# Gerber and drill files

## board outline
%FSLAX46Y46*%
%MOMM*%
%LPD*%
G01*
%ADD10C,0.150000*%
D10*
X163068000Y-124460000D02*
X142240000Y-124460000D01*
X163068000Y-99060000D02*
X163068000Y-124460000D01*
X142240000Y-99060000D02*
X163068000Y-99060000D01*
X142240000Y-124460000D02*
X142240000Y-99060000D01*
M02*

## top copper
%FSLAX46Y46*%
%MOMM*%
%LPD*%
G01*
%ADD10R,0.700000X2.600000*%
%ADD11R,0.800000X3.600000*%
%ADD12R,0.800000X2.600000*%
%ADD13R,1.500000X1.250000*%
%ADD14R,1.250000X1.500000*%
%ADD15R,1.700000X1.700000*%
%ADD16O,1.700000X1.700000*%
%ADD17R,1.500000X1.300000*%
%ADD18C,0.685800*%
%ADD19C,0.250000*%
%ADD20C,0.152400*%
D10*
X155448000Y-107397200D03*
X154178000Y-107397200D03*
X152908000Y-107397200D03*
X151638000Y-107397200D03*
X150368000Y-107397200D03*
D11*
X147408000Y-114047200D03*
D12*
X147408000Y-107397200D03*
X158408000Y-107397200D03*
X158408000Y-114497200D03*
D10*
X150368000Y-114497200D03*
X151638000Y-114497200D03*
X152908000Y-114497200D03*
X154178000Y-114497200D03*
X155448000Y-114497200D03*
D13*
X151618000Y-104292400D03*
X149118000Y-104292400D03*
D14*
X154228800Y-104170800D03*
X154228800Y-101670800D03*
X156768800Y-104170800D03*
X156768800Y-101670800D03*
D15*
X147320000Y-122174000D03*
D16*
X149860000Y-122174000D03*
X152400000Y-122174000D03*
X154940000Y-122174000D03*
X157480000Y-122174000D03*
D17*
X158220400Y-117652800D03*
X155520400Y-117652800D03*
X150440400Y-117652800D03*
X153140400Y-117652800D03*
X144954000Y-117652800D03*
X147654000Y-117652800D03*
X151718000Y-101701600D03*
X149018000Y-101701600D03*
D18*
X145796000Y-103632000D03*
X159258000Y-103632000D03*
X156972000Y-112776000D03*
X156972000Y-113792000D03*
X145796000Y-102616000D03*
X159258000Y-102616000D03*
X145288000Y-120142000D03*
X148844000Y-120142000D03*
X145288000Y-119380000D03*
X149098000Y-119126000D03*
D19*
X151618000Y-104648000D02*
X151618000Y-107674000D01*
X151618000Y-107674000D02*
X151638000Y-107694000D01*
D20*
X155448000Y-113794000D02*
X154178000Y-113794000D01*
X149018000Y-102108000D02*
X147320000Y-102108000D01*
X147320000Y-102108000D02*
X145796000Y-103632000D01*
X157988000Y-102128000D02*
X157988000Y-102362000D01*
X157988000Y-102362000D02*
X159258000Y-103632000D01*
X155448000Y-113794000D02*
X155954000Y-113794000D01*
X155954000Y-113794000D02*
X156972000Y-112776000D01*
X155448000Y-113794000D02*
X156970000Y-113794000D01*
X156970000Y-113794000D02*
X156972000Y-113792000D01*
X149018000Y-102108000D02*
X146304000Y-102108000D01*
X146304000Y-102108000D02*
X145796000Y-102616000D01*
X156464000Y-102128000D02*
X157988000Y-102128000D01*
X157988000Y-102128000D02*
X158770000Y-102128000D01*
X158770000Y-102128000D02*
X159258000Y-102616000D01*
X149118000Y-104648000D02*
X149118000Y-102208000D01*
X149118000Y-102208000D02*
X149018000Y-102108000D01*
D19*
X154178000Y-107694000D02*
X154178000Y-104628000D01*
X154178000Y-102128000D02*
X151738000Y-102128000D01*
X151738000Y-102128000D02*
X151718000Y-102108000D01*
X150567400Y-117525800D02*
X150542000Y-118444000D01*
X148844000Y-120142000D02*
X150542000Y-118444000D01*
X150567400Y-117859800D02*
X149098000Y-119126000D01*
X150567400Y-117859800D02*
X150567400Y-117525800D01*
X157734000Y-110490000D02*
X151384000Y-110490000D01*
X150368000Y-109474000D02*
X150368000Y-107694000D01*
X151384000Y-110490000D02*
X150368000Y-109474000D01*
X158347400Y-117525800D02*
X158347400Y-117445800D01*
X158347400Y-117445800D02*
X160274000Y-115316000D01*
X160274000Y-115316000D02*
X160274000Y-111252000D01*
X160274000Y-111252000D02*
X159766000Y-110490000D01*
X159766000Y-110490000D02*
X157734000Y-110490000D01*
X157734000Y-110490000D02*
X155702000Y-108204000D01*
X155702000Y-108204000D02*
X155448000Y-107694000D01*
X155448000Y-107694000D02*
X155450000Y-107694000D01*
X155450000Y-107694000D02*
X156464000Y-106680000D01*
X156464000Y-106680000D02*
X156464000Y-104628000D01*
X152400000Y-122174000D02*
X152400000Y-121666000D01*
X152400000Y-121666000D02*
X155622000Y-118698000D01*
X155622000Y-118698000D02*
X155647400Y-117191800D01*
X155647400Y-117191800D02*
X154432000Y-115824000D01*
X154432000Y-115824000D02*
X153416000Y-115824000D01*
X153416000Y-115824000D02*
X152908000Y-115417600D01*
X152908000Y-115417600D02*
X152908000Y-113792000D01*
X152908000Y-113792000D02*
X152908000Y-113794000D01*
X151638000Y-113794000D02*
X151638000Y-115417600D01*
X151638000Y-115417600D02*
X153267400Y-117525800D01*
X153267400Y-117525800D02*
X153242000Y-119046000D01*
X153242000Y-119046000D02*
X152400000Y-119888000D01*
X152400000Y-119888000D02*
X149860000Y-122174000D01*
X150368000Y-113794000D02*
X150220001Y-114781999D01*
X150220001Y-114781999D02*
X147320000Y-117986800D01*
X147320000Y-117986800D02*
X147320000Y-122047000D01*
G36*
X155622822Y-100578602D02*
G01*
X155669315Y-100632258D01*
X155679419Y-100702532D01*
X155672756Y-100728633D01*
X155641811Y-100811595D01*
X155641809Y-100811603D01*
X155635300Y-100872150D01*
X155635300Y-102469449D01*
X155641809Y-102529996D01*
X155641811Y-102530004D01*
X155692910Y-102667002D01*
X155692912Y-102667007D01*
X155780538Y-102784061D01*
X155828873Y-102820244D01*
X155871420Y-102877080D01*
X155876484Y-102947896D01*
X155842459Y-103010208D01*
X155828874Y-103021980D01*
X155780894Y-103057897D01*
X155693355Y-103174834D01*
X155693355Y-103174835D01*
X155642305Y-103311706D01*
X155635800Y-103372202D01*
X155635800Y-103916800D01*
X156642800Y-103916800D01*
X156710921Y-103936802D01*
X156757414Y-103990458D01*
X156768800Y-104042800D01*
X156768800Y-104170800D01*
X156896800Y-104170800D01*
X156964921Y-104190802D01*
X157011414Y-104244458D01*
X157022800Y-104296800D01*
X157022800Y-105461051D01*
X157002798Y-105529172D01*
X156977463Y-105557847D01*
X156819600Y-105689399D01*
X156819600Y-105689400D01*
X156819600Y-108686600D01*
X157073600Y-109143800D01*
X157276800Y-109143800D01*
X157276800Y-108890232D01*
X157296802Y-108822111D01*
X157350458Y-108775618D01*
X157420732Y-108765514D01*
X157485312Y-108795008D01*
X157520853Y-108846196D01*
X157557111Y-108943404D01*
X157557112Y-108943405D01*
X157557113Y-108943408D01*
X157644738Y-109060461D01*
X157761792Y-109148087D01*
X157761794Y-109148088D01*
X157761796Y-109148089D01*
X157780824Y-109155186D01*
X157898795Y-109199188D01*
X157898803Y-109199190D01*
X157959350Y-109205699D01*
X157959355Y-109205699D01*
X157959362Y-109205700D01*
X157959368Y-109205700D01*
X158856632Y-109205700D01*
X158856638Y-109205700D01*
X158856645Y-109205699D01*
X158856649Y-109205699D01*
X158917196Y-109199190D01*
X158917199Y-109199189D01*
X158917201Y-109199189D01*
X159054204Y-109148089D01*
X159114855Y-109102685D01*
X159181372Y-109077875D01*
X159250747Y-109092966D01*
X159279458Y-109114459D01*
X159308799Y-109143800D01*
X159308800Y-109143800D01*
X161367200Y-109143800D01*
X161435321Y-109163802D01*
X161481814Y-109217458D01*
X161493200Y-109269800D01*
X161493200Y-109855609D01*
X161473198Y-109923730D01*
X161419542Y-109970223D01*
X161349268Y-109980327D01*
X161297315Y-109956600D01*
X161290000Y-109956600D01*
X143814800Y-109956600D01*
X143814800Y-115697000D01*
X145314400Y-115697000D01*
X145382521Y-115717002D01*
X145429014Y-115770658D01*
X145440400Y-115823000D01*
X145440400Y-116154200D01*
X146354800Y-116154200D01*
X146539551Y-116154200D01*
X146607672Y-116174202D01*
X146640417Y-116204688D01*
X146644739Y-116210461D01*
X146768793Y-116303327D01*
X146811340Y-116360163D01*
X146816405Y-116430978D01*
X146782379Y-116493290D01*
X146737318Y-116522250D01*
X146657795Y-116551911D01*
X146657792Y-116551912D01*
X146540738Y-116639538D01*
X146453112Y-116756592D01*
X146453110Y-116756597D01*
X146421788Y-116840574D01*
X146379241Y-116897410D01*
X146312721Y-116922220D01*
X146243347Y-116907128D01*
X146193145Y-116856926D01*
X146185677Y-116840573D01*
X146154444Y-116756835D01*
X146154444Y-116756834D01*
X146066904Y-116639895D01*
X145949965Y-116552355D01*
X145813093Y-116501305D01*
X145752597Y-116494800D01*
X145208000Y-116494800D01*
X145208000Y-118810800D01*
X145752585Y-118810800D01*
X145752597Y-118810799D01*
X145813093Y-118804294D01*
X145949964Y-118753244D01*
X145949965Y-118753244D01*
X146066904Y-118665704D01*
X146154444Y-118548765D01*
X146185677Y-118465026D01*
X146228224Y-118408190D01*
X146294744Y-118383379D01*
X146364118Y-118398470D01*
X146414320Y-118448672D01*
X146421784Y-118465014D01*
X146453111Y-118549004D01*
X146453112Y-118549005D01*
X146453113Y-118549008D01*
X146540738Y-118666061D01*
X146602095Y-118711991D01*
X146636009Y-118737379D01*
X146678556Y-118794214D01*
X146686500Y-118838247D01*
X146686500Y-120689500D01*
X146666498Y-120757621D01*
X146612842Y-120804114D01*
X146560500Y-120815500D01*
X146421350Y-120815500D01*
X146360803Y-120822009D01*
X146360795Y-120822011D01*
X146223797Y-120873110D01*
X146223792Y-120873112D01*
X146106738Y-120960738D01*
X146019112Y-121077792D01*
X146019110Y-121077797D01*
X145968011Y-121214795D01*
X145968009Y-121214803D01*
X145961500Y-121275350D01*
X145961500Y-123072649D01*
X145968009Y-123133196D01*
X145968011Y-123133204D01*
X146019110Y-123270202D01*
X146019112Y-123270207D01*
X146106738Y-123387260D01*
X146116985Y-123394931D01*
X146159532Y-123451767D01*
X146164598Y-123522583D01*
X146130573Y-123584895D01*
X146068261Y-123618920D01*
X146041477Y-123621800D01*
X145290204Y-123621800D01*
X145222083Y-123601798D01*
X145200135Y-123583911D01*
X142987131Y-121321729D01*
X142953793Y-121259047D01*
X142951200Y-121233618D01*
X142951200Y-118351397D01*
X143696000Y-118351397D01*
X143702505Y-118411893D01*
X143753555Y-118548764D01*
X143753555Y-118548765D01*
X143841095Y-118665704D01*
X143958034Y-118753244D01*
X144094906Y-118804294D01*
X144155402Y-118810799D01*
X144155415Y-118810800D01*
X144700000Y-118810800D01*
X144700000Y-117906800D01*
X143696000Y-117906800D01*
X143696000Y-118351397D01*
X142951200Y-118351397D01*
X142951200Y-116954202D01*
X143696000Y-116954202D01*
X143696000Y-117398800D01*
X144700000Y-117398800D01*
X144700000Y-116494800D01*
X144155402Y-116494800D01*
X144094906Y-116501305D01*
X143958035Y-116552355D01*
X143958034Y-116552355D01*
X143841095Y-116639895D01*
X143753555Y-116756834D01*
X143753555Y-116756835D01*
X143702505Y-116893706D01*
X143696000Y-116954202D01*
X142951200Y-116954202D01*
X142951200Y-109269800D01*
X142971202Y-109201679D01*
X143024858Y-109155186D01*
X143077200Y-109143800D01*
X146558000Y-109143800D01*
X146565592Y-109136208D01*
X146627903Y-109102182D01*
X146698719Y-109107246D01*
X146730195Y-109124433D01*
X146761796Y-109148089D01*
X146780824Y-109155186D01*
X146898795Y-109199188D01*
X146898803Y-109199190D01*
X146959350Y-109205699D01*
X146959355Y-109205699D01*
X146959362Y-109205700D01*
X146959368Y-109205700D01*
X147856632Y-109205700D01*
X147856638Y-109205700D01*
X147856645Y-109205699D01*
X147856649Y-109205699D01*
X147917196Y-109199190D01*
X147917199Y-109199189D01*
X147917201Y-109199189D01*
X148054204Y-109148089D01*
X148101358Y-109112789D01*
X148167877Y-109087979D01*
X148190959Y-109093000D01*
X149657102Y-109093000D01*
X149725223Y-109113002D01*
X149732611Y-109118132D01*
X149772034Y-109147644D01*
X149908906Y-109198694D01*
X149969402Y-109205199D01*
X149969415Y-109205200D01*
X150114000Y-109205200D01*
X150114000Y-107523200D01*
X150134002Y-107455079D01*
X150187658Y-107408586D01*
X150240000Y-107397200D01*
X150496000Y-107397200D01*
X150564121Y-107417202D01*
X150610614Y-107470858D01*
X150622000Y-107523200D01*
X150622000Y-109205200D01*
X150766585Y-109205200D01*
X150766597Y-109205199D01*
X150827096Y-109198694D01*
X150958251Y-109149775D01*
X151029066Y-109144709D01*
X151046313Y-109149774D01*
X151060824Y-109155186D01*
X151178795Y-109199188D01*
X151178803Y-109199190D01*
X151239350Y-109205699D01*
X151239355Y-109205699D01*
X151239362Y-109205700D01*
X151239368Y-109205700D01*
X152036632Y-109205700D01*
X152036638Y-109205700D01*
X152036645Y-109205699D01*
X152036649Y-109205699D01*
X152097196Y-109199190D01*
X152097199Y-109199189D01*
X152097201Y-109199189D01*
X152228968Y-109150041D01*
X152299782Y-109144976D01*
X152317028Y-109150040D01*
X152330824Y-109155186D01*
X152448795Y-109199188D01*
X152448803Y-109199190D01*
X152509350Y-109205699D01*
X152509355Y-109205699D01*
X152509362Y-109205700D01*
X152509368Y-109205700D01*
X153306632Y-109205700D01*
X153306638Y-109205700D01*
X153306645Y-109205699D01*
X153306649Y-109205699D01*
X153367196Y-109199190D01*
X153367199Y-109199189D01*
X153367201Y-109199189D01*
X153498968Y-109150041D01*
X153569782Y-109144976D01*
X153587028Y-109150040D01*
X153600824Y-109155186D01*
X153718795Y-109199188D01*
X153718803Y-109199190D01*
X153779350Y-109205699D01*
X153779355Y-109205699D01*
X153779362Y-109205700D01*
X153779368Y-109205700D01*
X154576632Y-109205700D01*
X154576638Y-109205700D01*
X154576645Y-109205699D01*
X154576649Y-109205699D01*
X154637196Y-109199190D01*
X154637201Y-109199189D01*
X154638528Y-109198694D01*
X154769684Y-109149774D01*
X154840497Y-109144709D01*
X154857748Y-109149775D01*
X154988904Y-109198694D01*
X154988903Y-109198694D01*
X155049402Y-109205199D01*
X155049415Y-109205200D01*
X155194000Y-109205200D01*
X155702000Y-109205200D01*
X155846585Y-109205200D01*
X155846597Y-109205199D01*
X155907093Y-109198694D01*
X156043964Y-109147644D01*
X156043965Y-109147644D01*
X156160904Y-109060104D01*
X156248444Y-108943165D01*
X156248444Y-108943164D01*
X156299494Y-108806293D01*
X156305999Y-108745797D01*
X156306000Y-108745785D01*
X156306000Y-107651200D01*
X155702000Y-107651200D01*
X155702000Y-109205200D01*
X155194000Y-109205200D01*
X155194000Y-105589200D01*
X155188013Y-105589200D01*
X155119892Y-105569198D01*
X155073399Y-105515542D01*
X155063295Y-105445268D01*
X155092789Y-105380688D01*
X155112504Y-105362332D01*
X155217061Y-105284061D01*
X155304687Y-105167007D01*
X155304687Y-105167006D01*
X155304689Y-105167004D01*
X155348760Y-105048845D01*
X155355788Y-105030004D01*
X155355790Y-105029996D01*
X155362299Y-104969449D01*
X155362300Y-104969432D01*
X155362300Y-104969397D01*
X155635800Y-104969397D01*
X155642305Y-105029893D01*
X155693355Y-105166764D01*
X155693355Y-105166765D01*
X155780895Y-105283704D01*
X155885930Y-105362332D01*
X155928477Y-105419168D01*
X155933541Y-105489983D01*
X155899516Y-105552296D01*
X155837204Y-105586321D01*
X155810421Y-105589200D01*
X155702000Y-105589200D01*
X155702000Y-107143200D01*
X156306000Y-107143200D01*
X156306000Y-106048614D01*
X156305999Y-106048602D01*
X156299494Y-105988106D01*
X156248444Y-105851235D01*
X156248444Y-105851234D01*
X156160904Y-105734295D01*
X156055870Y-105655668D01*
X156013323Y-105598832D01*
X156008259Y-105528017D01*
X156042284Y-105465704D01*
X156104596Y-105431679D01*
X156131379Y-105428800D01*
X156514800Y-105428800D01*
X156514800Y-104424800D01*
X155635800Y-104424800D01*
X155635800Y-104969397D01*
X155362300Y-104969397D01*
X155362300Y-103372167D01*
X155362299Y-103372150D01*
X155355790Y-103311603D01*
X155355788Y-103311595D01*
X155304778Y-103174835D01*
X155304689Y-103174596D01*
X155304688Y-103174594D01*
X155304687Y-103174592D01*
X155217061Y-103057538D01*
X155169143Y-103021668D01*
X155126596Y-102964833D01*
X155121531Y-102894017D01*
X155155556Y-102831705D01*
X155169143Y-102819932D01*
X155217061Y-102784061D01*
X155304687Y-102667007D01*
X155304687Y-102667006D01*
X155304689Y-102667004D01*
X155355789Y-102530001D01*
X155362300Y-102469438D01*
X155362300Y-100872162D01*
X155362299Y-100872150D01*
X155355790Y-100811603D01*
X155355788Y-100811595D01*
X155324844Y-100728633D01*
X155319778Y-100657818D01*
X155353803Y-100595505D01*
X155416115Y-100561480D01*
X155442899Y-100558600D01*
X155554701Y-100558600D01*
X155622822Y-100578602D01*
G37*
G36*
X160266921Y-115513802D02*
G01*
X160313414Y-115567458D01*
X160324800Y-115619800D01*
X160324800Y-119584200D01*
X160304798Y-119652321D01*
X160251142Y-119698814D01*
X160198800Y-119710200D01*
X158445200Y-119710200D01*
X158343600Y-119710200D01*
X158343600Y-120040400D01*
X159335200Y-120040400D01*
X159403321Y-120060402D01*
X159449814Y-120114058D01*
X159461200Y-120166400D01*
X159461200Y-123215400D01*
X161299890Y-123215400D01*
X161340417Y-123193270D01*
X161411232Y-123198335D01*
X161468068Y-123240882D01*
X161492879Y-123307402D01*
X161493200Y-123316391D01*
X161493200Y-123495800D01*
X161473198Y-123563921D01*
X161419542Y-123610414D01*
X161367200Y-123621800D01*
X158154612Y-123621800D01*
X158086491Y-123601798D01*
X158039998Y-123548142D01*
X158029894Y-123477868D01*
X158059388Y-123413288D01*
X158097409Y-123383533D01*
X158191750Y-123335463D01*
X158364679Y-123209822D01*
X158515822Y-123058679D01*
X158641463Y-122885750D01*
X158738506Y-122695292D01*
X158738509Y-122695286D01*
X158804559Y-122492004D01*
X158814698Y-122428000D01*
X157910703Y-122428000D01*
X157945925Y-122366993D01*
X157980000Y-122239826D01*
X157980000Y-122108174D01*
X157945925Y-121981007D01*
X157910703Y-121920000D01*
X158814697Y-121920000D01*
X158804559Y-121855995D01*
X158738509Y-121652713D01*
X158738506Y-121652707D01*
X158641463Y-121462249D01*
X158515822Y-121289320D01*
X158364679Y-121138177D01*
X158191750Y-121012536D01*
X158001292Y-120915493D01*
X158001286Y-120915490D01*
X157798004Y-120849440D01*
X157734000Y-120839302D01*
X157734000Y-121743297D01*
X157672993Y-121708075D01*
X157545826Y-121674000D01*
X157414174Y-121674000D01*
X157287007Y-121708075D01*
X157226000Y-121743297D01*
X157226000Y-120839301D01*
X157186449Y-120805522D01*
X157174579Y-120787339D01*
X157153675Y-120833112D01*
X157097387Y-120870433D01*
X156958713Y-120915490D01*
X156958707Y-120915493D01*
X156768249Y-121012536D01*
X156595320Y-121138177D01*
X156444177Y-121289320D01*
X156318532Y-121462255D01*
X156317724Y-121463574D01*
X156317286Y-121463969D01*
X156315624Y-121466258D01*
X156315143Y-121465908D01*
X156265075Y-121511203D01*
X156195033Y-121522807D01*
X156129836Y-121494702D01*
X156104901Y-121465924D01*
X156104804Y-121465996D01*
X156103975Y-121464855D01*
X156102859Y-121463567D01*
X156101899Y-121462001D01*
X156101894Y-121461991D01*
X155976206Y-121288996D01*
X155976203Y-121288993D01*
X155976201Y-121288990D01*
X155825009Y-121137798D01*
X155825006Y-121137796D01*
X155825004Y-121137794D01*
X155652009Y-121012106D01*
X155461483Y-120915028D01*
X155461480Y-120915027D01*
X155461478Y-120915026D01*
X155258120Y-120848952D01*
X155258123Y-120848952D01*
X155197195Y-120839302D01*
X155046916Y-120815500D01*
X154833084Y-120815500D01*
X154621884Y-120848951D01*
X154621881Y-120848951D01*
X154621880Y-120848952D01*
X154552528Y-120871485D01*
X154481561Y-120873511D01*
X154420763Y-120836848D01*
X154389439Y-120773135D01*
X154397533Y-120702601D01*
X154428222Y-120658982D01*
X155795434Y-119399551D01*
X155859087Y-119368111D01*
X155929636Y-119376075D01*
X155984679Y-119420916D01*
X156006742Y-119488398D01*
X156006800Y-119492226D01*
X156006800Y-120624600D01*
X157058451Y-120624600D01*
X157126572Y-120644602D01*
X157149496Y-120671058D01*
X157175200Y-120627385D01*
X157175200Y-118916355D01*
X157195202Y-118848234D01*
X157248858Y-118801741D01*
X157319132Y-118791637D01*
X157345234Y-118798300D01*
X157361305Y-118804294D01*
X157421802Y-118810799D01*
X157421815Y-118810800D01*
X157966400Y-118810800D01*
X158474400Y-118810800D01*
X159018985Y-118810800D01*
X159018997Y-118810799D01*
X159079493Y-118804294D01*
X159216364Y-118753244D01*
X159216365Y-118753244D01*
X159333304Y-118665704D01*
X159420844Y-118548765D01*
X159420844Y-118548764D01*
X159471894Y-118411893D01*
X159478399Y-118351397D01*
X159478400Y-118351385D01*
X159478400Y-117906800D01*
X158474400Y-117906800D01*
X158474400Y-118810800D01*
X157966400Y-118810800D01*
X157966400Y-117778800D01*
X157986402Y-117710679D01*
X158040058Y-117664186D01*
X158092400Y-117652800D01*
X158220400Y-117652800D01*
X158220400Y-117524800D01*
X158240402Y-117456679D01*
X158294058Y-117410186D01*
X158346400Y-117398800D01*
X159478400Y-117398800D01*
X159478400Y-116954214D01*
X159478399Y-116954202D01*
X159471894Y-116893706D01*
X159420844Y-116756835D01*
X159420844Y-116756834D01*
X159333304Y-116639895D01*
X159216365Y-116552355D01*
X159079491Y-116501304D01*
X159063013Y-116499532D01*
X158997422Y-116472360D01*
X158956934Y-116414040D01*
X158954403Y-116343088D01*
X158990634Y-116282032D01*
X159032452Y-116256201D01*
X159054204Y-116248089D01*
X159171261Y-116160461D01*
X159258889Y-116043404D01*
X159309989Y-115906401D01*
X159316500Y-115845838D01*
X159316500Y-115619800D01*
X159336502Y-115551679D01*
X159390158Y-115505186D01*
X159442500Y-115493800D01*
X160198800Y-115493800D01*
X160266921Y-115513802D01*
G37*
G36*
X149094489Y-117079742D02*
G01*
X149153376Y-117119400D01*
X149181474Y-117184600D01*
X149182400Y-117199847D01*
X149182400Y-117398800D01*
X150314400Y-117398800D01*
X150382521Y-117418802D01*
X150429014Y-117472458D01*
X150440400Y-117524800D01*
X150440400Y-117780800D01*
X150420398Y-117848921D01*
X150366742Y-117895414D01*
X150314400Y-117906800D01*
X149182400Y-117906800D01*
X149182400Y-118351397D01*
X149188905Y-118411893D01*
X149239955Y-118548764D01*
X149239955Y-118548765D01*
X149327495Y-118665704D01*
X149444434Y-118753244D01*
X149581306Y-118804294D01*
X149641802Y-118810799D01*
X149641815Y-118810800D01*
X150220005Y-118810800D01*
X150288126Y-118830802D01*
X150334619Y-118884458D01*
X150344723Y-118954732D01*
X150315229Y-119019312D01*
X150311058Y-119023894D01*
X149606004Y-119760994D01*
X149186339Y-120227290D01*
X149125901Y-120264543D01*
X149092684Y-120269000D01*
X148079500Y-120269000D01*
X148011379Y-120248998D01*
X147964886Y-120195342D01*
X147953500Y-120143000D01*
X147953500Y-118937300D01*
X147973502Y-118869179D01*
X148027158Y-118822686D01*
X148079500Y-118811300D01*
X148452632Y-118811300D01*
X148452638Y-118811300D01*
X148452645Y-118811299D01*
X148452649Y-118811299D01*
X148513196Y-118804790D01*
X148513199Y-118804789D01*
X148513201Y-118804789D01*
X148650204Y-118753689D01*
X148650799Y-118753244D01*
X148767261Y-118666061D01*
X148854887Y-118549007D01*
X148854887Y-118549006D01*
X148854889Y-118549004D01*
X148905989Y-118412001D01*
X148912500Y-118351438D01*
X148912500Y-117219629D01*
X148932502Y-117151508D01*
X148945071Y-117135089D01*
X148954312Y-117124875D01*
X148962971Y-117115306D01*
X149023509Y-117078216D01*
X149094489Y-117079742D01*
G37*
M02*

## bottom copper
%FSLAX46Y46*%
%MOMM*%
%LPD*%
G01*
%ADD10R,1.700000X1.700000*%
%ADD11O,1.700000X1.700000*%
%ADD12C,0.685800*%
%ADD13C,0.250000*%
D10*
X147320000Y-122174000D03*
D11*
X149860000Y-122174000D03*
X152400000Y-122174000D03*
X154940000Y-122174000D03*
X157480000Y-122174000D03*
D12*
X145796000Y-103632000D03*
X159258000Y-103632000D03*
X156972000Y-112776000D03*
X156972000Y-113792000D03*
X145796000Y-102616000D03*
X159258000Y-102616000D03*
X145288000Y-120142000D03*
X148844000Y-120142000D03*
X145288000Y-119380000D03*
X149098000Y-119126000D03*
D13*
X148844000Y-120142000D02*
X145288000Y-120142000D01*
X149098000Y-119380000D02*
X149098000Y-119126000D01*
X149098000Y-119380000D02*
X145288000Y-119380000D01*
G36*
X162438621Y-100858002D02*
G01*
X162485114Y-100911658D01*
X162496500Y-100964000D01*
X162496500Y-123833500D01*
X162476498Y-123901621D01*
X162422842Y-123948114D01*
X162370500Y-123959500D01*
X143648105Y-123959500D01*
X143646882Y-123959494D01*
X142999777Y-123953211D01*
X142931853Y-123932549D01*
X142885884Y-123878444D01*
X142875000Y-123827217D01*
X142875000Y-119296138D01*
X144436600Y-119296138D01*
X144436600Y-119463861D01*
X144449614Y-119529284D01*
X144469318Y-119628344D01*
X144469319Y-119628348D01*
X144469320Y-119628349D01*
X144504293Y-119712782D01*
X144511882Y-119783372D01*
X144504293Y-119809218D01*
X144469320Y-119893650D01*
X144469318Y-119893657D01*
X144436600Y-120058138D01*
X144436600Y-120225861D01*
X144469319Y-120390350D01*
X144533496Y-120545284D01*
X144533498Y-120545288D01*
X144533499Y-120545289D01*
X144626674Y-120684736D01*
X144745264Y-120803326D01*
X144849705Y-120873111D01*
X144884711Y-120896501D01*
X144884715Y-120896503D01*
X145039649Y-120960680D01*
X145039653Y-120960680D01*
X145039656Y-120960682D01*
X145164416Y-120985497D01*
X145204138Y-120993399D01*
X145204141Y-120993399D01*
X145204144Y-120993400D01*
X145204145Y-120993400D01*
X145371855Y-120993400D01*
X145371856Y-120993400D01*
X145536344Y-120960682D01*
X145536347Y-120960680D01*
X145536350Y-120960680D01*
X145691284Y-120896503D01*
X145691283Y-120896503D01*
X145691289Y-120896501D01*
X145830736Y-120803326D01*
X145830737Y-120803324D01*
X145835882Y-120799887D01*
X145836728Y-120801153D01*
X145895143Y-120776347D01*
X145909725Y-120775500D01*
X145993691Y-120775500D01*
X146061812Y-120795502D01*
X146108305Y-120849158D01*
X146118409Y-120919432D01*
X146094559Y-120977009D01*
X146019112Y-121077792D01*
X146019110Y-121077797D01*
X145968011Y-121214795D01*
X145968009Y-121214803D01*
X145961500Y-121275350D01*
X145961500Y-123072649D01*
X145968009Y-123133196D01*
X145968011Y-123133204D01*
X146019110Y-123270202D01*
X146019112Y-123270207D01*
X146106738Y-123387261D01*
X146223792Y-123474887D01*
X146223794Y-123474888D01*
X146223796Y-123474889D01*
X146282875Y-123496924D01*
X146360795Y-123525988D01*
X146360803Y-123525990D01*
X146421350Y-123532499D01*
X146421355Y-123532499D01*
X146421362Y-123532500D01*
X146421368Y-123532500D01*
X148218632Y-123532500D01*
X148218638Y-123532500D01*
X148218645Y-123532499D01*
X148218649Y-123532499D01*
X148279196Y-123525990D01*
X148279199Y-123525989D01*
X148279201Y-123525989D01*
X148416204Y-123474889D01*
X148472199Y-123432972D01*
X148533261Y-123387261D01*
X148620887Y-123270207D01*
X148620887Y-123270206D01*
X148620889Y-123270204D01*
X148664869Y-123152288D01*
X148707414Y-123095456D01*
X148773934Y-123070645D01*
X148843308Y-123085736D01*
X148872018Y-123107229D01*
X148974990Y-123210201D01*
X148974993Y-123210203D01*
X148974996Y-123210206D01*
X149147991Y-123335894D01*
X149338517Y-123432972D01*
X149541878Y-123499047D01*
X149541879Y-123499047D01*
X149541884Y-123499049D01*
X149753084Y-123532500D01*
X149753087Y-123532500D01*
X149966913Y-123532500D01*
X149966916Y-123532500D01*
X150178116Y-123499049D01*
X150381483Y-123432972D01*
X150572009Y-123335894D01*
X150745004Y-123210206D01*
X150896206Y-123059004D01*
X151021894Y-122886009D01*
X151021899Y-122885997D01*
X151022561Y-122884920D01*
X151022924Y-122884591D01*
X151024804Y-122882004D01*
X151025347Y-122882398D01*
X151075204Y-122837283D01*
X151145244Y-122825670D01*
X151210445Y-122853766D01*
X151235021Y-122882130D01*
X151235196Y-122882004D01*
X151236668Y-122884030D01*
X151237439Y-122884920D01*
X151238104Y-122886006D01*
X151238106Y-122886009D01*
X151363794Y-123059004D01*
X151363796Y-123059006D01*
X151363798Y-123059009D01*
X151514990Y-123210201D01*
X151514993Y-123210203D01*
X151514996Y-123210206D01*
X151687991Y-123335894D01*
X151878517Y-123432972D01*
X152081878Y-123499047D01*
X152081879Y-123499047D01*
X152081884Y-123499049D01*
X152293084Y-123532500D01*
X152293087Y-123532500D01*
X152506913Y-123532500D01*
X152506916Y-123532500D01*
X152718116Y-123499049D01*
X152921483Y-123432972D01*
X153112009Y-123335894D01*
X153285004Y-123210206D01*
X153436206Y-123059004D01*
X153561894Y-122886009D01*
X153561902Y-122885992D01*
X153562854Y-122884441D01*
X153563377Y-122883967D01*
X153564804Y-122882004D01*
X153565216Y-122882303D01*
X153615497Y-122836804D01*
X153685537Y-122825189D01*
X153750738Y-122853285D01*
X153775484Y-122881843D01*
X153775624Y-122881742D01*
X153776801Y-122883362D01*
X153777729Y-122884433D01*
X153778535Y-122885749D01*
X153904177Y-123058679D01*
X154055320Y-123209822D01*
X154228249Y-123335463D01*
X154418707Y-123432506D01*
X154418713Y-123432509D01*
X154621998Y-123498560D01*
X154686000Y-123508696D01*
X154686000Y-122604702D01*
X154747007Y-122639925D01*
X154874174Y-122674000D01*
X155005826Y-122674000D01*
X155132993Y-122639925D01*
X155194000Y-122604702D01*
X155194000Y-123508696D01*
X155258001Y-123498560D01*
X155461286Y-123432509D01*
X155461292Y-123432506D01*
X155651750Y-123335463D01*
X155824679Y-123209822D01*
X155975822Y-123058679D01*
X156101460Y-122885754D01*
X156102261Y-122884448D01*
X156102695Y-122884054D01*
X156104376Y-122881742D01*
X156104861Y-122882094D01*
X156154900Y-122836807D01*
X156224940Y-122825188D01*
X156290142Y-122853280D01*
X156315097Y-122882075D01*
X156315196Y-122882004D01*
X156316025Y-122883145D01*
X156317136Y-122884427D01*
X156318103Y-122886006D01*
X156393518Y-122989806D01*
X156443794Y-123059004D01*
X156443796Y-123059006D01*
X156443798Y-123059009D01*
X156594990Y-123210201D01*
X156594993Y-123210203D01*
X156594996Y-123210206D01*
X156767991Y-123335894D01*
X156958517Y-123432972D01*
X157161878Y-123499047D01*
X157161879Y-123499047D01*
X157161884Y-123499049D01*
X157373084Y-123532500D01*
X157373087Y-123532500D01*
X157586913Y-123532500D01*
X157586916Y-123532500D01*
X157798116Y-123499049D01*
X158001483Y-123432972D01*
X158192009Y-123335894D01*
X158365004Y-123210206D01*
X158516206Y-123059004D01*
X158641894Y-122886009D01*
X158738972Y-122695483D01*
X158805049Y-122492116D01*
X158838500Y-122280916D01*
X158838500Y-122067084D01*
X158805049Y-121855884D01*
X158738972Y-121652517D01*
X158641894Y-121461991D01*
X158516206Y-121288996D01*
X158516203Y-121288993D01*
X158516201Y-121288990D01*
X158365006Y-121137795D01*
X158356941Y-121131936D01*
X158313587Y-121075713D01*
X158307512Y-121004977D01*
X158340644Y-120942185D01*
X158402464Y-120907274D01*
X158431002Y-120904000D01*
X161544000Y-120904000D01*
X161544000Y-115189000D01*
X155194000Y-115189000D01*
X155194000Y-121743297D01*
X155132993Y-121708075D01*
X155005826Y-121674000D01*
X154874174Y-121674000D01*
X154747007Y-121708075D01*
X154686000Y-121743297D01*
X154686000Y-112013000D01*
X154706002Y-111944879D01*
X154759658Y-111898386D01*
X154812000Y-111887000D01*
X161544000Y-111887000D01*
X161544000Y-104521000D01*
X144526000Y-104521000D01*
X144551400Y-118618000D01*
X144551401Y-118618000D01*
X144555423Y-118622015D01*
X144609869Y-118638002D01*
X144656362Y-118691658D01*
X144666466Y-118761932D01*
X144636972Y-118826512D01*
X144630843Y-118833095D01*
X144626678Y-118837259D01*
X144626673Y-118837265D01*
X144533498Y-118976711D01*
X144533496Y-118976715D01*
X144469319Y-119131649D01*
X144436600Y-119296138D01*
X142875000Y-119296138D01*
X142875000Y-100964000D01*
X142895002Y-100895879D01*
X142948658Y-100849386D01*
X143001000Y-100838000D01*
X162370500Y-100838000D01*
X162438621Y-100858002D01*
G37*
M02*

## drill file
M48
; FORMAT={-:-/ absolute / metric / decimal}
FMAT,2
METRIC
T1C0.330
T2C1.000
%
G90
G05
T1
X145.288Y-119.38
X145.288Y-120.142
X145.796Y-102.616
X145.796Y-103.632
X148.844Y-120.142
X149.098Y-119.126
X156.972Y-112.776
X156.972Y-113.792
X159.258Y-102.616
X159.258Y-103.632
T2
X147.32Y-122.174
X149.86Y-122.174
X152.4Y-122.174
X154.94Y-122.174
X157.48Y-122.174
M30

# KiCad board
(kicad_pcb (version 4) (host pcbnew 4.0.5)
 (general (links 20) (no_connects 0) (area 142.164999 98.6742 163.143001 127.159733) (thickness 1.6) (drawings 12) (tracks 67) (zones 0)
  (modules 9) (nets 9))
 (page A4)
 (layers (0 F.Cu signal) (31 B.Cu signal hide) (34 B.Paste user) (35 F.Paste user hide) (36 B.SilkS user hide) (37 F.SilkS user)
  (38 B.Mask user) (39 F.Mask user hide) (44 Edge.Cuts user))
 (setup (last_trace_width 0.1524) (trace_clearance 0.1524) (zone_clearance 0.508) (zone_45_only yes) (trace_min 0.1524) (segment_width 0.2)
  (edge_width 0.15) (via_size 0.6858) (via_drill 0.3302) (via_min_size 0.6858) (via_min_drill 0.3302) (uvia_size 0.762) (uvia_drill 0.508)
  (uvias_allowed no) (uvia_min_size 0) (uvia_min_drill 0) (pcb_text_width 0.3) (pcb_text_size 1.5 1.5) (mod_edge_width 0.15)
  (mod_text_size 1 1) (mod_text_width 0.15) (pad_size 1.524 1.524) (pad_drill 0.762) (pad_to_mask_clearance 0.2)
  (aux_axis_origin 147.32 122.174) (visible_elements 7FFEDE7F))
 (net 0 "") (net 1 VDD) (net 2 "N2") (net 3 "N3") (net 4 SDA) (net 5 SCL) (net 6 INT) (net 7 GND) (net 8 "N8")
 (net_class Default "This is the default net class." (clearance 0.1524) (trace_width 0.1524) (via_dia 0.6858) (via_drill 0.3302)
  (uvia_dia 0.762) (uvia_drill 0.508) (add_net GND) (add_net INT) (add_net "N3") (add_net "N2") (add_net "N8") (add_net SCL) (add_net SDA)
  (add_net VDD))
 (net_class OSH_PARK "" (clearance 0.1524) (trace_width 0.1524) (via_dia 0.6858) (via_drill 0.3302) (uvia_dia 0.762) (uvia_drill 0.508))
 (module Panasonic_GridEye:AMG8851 (layer F.Cu) (at 152.908 110.9472)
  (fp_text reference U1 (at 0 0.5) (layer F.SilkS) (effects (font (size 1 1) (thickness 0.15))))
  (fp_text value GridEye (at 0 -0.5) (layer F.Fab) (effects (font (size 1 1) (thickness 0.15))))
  (pad 9 smd rect (at 2.54 -3.55) (size 0.7 2.6) (layers F.Cu F.Paste F.Mask) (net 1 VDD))
  (pad 10 smd rect (at 1.27 -3.55) (size 0.7 2.6) (layers F.Cu F.Paste F.Mask) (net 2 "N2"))
  (pad 11 smd rect (at 0 -3.55) (size 0.7 2.6) (layers F.Cu F.Paste F.Mask))
  (pad 12 smd rect (at -1.27 -3.55) (size 0.7 2.6) (layers F.Cu F.Paste F.Mask) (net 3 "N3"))
  (pad 13 smd rect (at -2.54 -3.55) (size 0.7 2.6) (layers F.Cu F.Paste F.Mask) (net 1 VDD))
  (pad 1 smd rect (at -5.5 3.1) (size 0.8 3.6) (layers F.Cu F.Paste F.Mask))
  (pad 14 smd rect (at -5.5 -3.55) (size 0.8 2.6) (layers F.Cu F.Paste F.Mask))
  (pad 8 smd rect (at 5.5 -3.55) (size 0.8 2.6) (layers F.Cu F.Paste F.Mask))
  (pad 7 smd rect (at 5.5 3.55) (size 0.8 2.6) (layers F.Cu F.Paste F.Mask))
  (pad 2 smd rect (at -2.54 3.55) (size 0.7 2.6) (layers F.Cu F.Paste F.Mask) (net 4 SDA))
  (pad 3 smd rect (at -1.27 3.55) (size 0.7 2.6) (layers F.Cu F.Paste F.Mask) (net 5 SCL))
  (pad 4 smd rect (at 0 3.55) (size 0.7 2.6) (layers F.Cu F.Paste F.Mask) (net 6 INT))
  (pad 5 smd rect (at 1.27 3.55) (size 0.7 2.6) (layers F.Cu F.Paste F.Mask) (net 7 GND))
  (pad 6 smd rect (at 2.54 3.55) (size 0.7 2.6) (layers F.Cu F.Paste F.Mask) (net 7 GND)))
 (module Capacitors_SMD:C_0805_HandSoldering (layer F.Cu) (at 150.368 104.2924 180)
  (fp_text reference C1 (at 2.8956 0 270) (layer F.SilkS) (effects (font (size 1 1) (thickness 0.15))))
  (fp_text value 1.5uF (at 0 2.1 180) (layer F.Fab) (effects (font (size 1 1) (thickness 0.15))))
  (pad 1 smd rect (at -1.25 0 180) (size 1.5 1.25) (layers F.Cu F.Paste F.Mask) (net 3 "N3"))
  (pad 2 smd rect (at 1.25 0 180) (size 1.5 1.25) (layers F.Cu F.Paste F.Mask) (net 7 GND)))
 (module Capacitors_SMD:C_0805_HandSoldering (layer F.Cu) (at 154.2288 102.9208 90)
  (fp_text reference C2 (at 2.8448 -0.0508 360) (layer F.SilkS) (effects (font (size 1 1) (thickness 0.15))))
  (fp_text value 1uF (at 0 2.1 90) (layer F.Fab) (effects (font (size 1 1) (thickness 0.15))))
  (pad 1 smd rect (at -1.25 0 90) (size 1.5 1.25) (layers F.Cu F.Paste F.Mask) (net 2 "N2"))
  (pad 2 smd rect (at 1.25 0 90) (size 1.5 1.25) (layers F.Cu F.Paste F.Mask) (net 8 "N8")))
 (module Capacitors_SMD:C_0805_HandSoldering (layer F.Cu) (at 156.7688 102.9208 90)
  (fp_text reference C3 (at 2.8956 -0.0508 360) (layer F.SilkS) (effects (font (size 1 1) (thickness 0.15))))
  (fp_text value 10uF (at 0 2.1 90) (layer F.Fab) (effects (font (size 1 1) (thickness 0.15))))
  (pad 1 smd rect (at -1.25 0 90) (size 1.5 1.25) (layers F.Cu F.Paste F.Mask) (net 1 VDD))
  (pad 2 smd rect (at 1.25 0 90) (size 1.5 1.25) (layers F.Cu F.Paste F.Mask) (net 7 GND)))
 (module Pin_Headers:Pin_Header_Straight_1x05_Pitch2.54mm (layer F.Cu) (at 147.32 122.174 90)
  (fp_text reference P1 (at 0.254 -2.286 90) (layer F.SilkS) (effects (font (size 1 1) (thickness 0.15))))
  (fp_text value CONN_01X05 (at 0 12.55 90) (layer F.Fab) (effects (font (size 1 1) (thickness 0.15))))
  (pad 1 thru_hole rect (at 0 0 90) (size 1.7 1.7) (drill 1) (layers *.Cu *.Mask) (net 4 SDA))
  (pad 2 thru_hole oval (at 0 2.54 90) (size 1.7 1.7) (drill 1) (layers *.Cu *.Mask) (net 5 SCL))
  (pad 3 thru_hole oval (at 0 5.08 90) (size 1.7 1.7) (drill 1) (layers *.Cu *.Mask) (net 6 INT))
  (pad 4 thru_hole oval (at 0 7.62 90) (size 1.7 1.7) (drill 1) (layers *.Cu *.Mask) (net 7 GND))
  (pad 5 thru_hole oval (at 0 10.16 90) (size 1.7 1.7) (drill 1) (layers *.Cu *.Mask) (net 1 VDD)))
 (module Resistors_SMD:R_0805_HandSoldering (layer F.Cu) (at 156.8704 117.6528 180)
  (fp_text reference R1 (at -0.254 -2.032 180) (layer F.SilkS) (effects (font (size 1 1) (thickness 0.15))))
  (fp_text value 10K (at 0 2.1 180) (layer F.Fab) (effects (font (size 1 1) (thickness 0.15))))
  (pad 1 smd rect (at -1.35 0 180) (size 1.5 1.3) (layers F.Cu F.Paste F.Mask) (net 1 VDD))
  (pad 2 smd rect (at 1.35 0 180) (size 1.5 1.3) (layers F.Cu F.Paste F.Mask) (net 6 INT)))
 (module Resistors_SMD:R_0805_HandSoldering (layer F.Cu) (at 151.7904 117.6528)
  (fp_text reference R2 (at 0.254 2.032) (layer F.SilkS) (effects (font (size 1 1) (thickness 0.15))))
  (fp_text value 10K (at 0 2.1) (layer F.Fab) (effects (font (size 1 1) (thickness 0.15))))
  (pad 1 smd rect (at -1.35 0) (size 1.5 1.3) (layers F.Cu F.Paste F.Mask) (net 1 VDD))
  (pad 2 smd rect (at 1.35 0) (size 1.5 1.3) (layers F.Cu F.Paste F.Mask) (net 5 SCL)))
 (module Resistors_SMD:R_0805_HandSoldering (layer F.Cu) (at 146.304 117.6528)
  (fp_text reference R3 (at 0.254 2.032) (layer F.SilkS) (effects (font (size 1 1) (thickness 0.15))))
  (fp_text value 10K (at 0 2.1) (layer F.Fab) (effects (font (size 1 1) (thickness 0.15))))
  (pad 1 smd rect (at -1.35 0) (size 1.5 1.3) (layers F.Cu F.Paste F.Mask) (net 1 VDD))
  (pad 2 smd rect (at 1.35 0) (size 1.5 1.3) (layers F.Cu F.Paste F.Mask) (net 4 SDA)))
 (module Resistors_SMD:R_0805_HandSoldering (layer F.Cu) (at 150.368 101.7016 180)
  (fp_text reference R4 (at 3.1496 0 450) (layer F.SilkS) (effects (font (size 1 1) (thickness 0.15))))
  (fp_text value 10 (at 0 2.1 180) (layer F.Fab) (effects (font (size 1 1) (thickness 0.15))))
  (pad 1 smd rect (at -1.35 0 180) (size 1.5 1.3) (layers F.Cu F.Paste F.Mask) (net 8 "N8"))
  (pad 2 smd rect (at 1.35 0 180) (size 1.5 1.3) (layers F.Cu F.Paste F.Mask) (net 7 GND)))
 (gr_line (start 163.068 124.46) (end 142.24 124.46) (angle 90) (layer Edge.Cuts) (width 0.15))
 (gr_line (start 163.068 99.06) (end 163.068 124.46) (angle 90) (layer Edge.Cuts) (width 0.15))
 (gr_line (start 142.24 99.06) (end 163.068 99.06) (angle 90) (layer Edge.Cuts) (width 0.15))
 (gr_line (start 142.24 124.46) (end 142.24 99.06) (angle 90) (layer Edge.Cuts) (width 0.15))
 (segment (start 151.618 104.648) (end 151.618 107.674) (width 0.25) (layer F.Cu) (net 3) (status 20))
 (segment (start 151.618 107.674) (end 151.638 107.694) (width 0.25) (layer F.Cu) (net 3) (status 30))
 (segment (start 155.448 113.794) (end 154.178 113.794) (width 0.1524) (layer F.Cu) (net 7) (status 30))
 (via (at 145.796 103.632) (size 0.6858) (drill 0.3302) (layers F.Cu B.Cu) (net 7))
 (segment (start 149.018 102.108) (end 147.32 102.108) (width 0.1524) (layer F.Cu) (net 7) (status 10))
 (segment (start 147.32 102.108) (end 145.796 103.632) (width 0.1524) (layer F.Cu) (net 7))
 (via (at 159.258 103.632) (size 0.6858) (drill 0.3302) (layers F.Cu B.Cu) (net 7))
 (segment (start 157.988 102.128) (end 157.988 102.362) (width 0.1524) (layer F.Cu) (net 7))
 (segment (start 157.988 102.362) (end 159.258 103.632) (width 0.1524) (layer F.Cu) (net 7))
 (via (at 156.972 112.776) (size 0.6858) (drill 0.3302) (layers F.Cu B.Cu) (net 7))
 (segment (start 155.448 113.794) (end 155.954 113.794) (width 0.1524) (layer F.Cu) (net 7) (status 10))
 (segment (start 155.954 113.794) (end 156.972 112.776) (width 0.1524) (layer F.Cu) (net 7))
 (via (at 156.972 113.792) (size 0.6858) (drill 0.3302) (layers F.Cu B.Cu) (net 7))
 (segment (start 155.448 113.794) (end 156.97 113.794) (width 0.1524) (layer F.Cu) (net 7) (status 10))
 (segment (start 156.97 113.794) (end 156.972 113.792) (width 0.1524) (layer F.Cu) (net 7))
 (via (at 145.796 102.616) (size 0.6858) (drill 0.3302) (layers F.Cu B.Cu) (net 7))
 (segment (start 149.018 102.108) (end 146.304 102.108) (width 0.1524) (layer F.Cu) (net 7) (status 10))
 (segment (start 146.304 102.108) (end 145.796 102.616) (width 0.1524) (layer F.Cu) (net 7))
 (via (at 159.258 102.616) (size 0.6858) (drill 0.3302) (layers F.Cu B.Cu) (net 7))
 (segment (start 156.464 102.128) (end 157.988 102.128) (width 0.1524) (layer F.Cu) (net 7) (status 10))
 (segment (start 157.988 102.128) (end 158.77 102.128) (width 0.1524) (layer F.Cu) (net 7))
 (segment (start 158.77 102.128) (end 159.258 102.616) (width 0.1524) (layer F.Cu) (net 7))
 (segment (start 149.118 104.648) (end 149.118 102.208) (width 0.1524) (layer F.Cu) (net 7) (status 30))
 (segment (start 149.118 102.208) (end 149.018 102.108) (width 0.1524) (layer F.Cu) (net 7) (status 30))
 (segment (start 154.178 107.694) (end 154.178 104.628) (width 0.25) (layer F.Cu) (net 2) (status 10))
 (segment (start 154.178 102.128) (end 151.738 102.128) (width 0.25) (layer F.Cu) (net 8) (status 30))
 (segment (start 151.738 102.128) (end 151.718 102.108) (width 0.25) (layer F.Cu) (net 8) (status 30))
 (via (at 145.288 120.142) (size 0.6858) (drill 0.3302) (layers F.Cu B.Cu) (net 1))
 (segment (start 150.5674 117.5258) (end 150.542 118.444) (width 0.25) (layer F.Cu) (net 1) (status 10))
 (segment (start 148.844 120.142) (end 150.542 118.444) (width 0.25) (layer F.Cu) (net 1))
 (via (at 148.844 120.142) (size 0.6858) (drill 0.3302) (layers F.Cu B.Cu) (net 1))
 (segment (start 148.844 120.142) (end 145.288 120.142) (width 0.25) (layer B.Cu) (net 1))
 (via (at 145.288 119.38) (size 0.6858) (drill 0.3302) (layers F.Cu B.Cu) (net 1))
 (segment (start 150.5674 117.8598) (end 149.098 119.126) (width 0.25) (layer F.Cu) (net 1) (status 10))
 (via (at 149.098 119.126) (size 0.6858) (drill 0.3302) (layers F.Cu B.Cu) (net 1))
 (segment (start 149.098 119.38) (end 149.098 119.126) (width 0.25) (layer B.Cu) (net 1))
 (segment (start 149.098 119.38) (end 145.288 119.38) (width 0.25) (layer B.Cu) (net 1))
 (segment (start 150.5674 117.8598) (end 150.5674 117.5258) (width 0.25) (layer F.Cu) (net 1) (status 30))
 (segment (start 157.734 110.49) (end 151.384 110.49) (width 0.25) (layer F.Cu) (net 1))
 (segment (start 150.368 109.474) (end 150.368 107.694) (width 0.25) (layer F.Cu) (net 1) (status 20))
 (segment (start 151.384 110.49) (end 150.368 109.474) (width 0.25) (layer F.Cu) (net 1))
 (segment (start 158.3474 117.5258) (end 158.3474 117.4458) (width 0.25) (layer F.Cu) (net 1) (status 30))
 (segment (start 158.3474 117.4458) (end 160.274 115.316) (width 0.25) (layer F.Cu) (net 1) (status 10))
 (segment (start 160.274 115.316) (end 160.274 111.252) (width 0.25) (layer F.Cu) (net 1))
 (segment (start 160.274 111.252) (end 159.766 110.49) (width 0.25) (layer F.Cu) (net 1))
 (segment (start 159.766 110.49) (end 157.734 110.49) (width 0.25) (layer F.Cu) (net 1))
 (segment (start 157.734 110.49) (end 155.702 108.204) (width 0.25) (layer F.Cu) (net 1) (status 20))
 (segment (start 155.702 108.204) (end 155.448 107.694) (width 0.25) (layer F.Cu) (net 1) (status 30))
 (segment (start 155.448 107.694) (end 155.45 107.694) (width 0.25) (layer F.Cu) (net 1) (status 30))
 (segment (start 155.45 107.694) (end 156.464 106.68) (width 0.25) (layer F.Cu) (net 1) (status 10))
 (segment (start 156.464 106.68) (end 156.464 104.628) (width 0.25) (layer F.Cu) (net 1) (status 20))
 (segment (start 152.4 122.174) (end 152.4 121.666) (width 0.25) (layer F.Cu) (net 6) (status 30))
 (segment (start 152.4 121.666) (end 155.622 118.698) (width 0.25) (layer F.Cu) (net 6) (status 10))
 (segment (start 155.622 118.698) (end 155.6474 117.1918) (width 0.25) (layer F.Cu) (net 6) (status 20))
 (segment (start 155.6474 117.1918) (end 154.432 115.824) (width 0.25) (layer F.Cu) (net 6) (status 10))
 (segment (start 154.432 115.824) (end 153.416 115.824) (width 0.25) (layer F.Cu) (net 6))
 (segment (start 153.416 115.824) (end 152.908 115.4176) (width 0.25) (layer F.Cu) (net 6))
 (segment (start 152.908 115.4176) (end 152.908 113.792) (width 0.25) (layer F.Cu) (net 6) (status 20))
 (segment (start 152.908 113.792) (end 152.908 113.794) (width 0.25) (layer F.Cu) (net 6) (status 30))
 (segment (start 151.638 113.794) (end 151.638 115.4176) (width 0.25) (layer F.Cu) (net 5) (status 10))
 (segment (start 151.638 115.4176) (end 153.2674 117.5258) (width 0.25) (layer F.Cu) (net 5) (status 20))
 (segment (start 153.2674 117.5258) (end 153.242 119.046) (width 0.25) (layer F.Cu) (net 5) (status 10))
 (segment (start 153.242 119.046) (end 152.4 119.888) (width 0.25) (layer F.Cu) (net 5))
 (segment (start 152.4 119.888) (end 149.86 122.174) (width 0.25) (layer F.Cu) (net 5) (status 20))
 (segment (start 150.368 113.794) (end 150.220001 114.781999) (width 0.25) (layer F.Cu) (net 4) (status 30))
 (segment (start 150.220001 114.781999) (end 147.32 117.9868) (width 0.25) (layer F.Cu) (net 4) (status 20))
 (segment (start 147.32 117.9868) (end 147.32 122.047) (width 0.25) (layer F.Cu) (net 4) (status 10))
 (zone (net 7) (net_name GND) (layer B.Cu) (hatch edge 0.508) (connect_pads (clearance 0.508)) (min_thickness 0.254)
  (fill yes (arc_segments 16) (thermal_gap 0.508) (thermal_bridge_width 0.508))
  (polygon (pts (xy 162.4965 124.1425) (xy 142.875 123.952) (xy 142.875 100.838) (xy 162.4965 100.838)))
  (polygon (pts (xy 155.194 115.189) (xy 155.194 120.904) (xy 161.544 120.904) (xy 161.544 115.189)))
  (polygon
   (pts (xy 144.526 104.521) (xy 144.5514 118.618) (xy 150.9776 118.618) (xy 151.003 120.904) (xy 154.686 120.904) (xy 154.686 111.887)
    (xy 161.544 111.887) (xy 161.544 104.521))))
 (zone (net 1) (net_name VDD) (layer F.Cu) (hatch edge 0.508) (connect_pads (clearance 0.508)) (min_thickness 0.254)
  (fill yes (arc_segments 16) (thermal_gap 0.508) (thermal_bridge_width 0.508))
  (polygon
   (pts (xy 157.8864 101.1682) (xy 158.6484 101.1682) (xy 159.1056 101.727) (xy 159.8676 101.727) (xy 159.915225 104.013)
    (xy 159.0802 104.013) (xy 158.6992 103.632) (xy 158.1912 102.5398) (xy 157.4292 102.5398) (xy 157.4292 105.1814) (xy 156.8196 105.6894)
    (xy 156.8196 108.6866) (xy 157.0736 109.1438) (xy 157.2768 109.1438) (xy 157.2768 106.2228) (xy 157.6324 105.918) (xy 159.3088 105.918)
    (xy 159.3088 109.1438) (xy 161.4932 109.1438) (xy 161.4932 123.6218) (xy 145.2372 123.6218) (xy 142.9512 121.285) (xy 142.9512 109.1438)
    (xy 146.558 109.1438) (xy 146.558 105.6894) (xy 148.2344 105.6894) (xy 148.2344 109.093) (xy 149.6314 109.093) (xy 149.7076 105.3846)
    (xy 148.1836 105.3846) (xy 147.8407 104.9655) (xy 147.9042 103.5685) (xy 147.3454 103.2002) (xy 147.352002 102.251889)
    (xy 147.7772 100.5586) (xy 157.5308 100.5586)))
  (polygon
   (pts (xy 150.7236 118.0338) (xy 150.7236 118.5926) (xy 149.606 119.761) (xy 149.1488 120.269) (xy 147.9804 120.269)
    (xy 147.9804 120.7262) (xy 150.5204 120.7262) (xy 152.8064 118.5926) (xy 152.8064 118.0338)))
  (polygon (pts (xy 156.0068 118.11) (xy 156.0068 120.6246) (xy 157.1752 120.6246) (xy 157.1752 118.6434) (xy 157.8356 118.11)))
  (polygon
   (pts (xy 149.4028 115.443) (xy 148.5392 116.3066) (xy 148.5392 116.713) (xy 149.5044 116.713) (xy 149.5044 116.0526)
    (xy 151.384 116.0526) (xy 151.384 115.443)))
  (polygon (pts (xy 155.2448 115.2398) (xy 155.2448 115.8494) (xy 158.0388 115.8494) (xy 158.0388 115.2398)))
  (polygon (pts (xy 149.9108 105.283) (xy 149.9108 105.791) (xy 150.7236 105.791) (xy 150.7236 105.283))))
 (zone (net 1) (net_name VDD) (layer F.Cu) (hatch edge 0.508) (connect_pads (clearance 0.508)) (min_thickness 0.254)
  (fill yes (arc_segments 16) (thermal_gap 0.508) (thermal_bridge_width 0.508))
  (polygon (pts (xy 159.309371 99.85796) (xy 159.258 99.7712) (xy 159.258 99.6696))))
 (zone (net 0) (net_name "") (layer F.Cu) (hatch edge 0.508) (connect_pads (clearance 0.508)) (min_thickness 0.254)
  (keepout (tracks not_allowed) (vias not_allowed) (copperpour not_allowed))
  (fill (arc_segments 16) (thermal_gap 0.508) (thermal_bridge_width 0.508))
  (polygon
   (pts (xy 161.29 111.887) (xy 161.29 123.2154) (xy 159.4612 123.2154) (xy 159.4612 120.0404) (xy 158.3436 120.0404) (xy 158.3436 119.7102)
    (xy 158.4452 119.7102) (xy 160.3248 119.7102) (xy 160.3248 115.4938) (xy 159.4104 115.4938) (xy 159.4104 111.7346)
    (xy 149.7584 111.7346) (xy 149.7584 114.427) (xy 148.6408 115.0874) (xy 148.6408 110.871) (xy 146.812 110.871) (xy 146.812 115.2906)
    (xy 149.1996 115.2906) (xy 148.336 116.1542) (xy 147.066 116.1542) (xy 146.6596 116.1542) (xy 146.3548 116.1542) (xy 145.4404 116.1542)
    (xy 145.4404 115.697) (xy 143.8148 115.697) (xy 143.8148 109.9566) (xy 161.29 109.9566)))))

